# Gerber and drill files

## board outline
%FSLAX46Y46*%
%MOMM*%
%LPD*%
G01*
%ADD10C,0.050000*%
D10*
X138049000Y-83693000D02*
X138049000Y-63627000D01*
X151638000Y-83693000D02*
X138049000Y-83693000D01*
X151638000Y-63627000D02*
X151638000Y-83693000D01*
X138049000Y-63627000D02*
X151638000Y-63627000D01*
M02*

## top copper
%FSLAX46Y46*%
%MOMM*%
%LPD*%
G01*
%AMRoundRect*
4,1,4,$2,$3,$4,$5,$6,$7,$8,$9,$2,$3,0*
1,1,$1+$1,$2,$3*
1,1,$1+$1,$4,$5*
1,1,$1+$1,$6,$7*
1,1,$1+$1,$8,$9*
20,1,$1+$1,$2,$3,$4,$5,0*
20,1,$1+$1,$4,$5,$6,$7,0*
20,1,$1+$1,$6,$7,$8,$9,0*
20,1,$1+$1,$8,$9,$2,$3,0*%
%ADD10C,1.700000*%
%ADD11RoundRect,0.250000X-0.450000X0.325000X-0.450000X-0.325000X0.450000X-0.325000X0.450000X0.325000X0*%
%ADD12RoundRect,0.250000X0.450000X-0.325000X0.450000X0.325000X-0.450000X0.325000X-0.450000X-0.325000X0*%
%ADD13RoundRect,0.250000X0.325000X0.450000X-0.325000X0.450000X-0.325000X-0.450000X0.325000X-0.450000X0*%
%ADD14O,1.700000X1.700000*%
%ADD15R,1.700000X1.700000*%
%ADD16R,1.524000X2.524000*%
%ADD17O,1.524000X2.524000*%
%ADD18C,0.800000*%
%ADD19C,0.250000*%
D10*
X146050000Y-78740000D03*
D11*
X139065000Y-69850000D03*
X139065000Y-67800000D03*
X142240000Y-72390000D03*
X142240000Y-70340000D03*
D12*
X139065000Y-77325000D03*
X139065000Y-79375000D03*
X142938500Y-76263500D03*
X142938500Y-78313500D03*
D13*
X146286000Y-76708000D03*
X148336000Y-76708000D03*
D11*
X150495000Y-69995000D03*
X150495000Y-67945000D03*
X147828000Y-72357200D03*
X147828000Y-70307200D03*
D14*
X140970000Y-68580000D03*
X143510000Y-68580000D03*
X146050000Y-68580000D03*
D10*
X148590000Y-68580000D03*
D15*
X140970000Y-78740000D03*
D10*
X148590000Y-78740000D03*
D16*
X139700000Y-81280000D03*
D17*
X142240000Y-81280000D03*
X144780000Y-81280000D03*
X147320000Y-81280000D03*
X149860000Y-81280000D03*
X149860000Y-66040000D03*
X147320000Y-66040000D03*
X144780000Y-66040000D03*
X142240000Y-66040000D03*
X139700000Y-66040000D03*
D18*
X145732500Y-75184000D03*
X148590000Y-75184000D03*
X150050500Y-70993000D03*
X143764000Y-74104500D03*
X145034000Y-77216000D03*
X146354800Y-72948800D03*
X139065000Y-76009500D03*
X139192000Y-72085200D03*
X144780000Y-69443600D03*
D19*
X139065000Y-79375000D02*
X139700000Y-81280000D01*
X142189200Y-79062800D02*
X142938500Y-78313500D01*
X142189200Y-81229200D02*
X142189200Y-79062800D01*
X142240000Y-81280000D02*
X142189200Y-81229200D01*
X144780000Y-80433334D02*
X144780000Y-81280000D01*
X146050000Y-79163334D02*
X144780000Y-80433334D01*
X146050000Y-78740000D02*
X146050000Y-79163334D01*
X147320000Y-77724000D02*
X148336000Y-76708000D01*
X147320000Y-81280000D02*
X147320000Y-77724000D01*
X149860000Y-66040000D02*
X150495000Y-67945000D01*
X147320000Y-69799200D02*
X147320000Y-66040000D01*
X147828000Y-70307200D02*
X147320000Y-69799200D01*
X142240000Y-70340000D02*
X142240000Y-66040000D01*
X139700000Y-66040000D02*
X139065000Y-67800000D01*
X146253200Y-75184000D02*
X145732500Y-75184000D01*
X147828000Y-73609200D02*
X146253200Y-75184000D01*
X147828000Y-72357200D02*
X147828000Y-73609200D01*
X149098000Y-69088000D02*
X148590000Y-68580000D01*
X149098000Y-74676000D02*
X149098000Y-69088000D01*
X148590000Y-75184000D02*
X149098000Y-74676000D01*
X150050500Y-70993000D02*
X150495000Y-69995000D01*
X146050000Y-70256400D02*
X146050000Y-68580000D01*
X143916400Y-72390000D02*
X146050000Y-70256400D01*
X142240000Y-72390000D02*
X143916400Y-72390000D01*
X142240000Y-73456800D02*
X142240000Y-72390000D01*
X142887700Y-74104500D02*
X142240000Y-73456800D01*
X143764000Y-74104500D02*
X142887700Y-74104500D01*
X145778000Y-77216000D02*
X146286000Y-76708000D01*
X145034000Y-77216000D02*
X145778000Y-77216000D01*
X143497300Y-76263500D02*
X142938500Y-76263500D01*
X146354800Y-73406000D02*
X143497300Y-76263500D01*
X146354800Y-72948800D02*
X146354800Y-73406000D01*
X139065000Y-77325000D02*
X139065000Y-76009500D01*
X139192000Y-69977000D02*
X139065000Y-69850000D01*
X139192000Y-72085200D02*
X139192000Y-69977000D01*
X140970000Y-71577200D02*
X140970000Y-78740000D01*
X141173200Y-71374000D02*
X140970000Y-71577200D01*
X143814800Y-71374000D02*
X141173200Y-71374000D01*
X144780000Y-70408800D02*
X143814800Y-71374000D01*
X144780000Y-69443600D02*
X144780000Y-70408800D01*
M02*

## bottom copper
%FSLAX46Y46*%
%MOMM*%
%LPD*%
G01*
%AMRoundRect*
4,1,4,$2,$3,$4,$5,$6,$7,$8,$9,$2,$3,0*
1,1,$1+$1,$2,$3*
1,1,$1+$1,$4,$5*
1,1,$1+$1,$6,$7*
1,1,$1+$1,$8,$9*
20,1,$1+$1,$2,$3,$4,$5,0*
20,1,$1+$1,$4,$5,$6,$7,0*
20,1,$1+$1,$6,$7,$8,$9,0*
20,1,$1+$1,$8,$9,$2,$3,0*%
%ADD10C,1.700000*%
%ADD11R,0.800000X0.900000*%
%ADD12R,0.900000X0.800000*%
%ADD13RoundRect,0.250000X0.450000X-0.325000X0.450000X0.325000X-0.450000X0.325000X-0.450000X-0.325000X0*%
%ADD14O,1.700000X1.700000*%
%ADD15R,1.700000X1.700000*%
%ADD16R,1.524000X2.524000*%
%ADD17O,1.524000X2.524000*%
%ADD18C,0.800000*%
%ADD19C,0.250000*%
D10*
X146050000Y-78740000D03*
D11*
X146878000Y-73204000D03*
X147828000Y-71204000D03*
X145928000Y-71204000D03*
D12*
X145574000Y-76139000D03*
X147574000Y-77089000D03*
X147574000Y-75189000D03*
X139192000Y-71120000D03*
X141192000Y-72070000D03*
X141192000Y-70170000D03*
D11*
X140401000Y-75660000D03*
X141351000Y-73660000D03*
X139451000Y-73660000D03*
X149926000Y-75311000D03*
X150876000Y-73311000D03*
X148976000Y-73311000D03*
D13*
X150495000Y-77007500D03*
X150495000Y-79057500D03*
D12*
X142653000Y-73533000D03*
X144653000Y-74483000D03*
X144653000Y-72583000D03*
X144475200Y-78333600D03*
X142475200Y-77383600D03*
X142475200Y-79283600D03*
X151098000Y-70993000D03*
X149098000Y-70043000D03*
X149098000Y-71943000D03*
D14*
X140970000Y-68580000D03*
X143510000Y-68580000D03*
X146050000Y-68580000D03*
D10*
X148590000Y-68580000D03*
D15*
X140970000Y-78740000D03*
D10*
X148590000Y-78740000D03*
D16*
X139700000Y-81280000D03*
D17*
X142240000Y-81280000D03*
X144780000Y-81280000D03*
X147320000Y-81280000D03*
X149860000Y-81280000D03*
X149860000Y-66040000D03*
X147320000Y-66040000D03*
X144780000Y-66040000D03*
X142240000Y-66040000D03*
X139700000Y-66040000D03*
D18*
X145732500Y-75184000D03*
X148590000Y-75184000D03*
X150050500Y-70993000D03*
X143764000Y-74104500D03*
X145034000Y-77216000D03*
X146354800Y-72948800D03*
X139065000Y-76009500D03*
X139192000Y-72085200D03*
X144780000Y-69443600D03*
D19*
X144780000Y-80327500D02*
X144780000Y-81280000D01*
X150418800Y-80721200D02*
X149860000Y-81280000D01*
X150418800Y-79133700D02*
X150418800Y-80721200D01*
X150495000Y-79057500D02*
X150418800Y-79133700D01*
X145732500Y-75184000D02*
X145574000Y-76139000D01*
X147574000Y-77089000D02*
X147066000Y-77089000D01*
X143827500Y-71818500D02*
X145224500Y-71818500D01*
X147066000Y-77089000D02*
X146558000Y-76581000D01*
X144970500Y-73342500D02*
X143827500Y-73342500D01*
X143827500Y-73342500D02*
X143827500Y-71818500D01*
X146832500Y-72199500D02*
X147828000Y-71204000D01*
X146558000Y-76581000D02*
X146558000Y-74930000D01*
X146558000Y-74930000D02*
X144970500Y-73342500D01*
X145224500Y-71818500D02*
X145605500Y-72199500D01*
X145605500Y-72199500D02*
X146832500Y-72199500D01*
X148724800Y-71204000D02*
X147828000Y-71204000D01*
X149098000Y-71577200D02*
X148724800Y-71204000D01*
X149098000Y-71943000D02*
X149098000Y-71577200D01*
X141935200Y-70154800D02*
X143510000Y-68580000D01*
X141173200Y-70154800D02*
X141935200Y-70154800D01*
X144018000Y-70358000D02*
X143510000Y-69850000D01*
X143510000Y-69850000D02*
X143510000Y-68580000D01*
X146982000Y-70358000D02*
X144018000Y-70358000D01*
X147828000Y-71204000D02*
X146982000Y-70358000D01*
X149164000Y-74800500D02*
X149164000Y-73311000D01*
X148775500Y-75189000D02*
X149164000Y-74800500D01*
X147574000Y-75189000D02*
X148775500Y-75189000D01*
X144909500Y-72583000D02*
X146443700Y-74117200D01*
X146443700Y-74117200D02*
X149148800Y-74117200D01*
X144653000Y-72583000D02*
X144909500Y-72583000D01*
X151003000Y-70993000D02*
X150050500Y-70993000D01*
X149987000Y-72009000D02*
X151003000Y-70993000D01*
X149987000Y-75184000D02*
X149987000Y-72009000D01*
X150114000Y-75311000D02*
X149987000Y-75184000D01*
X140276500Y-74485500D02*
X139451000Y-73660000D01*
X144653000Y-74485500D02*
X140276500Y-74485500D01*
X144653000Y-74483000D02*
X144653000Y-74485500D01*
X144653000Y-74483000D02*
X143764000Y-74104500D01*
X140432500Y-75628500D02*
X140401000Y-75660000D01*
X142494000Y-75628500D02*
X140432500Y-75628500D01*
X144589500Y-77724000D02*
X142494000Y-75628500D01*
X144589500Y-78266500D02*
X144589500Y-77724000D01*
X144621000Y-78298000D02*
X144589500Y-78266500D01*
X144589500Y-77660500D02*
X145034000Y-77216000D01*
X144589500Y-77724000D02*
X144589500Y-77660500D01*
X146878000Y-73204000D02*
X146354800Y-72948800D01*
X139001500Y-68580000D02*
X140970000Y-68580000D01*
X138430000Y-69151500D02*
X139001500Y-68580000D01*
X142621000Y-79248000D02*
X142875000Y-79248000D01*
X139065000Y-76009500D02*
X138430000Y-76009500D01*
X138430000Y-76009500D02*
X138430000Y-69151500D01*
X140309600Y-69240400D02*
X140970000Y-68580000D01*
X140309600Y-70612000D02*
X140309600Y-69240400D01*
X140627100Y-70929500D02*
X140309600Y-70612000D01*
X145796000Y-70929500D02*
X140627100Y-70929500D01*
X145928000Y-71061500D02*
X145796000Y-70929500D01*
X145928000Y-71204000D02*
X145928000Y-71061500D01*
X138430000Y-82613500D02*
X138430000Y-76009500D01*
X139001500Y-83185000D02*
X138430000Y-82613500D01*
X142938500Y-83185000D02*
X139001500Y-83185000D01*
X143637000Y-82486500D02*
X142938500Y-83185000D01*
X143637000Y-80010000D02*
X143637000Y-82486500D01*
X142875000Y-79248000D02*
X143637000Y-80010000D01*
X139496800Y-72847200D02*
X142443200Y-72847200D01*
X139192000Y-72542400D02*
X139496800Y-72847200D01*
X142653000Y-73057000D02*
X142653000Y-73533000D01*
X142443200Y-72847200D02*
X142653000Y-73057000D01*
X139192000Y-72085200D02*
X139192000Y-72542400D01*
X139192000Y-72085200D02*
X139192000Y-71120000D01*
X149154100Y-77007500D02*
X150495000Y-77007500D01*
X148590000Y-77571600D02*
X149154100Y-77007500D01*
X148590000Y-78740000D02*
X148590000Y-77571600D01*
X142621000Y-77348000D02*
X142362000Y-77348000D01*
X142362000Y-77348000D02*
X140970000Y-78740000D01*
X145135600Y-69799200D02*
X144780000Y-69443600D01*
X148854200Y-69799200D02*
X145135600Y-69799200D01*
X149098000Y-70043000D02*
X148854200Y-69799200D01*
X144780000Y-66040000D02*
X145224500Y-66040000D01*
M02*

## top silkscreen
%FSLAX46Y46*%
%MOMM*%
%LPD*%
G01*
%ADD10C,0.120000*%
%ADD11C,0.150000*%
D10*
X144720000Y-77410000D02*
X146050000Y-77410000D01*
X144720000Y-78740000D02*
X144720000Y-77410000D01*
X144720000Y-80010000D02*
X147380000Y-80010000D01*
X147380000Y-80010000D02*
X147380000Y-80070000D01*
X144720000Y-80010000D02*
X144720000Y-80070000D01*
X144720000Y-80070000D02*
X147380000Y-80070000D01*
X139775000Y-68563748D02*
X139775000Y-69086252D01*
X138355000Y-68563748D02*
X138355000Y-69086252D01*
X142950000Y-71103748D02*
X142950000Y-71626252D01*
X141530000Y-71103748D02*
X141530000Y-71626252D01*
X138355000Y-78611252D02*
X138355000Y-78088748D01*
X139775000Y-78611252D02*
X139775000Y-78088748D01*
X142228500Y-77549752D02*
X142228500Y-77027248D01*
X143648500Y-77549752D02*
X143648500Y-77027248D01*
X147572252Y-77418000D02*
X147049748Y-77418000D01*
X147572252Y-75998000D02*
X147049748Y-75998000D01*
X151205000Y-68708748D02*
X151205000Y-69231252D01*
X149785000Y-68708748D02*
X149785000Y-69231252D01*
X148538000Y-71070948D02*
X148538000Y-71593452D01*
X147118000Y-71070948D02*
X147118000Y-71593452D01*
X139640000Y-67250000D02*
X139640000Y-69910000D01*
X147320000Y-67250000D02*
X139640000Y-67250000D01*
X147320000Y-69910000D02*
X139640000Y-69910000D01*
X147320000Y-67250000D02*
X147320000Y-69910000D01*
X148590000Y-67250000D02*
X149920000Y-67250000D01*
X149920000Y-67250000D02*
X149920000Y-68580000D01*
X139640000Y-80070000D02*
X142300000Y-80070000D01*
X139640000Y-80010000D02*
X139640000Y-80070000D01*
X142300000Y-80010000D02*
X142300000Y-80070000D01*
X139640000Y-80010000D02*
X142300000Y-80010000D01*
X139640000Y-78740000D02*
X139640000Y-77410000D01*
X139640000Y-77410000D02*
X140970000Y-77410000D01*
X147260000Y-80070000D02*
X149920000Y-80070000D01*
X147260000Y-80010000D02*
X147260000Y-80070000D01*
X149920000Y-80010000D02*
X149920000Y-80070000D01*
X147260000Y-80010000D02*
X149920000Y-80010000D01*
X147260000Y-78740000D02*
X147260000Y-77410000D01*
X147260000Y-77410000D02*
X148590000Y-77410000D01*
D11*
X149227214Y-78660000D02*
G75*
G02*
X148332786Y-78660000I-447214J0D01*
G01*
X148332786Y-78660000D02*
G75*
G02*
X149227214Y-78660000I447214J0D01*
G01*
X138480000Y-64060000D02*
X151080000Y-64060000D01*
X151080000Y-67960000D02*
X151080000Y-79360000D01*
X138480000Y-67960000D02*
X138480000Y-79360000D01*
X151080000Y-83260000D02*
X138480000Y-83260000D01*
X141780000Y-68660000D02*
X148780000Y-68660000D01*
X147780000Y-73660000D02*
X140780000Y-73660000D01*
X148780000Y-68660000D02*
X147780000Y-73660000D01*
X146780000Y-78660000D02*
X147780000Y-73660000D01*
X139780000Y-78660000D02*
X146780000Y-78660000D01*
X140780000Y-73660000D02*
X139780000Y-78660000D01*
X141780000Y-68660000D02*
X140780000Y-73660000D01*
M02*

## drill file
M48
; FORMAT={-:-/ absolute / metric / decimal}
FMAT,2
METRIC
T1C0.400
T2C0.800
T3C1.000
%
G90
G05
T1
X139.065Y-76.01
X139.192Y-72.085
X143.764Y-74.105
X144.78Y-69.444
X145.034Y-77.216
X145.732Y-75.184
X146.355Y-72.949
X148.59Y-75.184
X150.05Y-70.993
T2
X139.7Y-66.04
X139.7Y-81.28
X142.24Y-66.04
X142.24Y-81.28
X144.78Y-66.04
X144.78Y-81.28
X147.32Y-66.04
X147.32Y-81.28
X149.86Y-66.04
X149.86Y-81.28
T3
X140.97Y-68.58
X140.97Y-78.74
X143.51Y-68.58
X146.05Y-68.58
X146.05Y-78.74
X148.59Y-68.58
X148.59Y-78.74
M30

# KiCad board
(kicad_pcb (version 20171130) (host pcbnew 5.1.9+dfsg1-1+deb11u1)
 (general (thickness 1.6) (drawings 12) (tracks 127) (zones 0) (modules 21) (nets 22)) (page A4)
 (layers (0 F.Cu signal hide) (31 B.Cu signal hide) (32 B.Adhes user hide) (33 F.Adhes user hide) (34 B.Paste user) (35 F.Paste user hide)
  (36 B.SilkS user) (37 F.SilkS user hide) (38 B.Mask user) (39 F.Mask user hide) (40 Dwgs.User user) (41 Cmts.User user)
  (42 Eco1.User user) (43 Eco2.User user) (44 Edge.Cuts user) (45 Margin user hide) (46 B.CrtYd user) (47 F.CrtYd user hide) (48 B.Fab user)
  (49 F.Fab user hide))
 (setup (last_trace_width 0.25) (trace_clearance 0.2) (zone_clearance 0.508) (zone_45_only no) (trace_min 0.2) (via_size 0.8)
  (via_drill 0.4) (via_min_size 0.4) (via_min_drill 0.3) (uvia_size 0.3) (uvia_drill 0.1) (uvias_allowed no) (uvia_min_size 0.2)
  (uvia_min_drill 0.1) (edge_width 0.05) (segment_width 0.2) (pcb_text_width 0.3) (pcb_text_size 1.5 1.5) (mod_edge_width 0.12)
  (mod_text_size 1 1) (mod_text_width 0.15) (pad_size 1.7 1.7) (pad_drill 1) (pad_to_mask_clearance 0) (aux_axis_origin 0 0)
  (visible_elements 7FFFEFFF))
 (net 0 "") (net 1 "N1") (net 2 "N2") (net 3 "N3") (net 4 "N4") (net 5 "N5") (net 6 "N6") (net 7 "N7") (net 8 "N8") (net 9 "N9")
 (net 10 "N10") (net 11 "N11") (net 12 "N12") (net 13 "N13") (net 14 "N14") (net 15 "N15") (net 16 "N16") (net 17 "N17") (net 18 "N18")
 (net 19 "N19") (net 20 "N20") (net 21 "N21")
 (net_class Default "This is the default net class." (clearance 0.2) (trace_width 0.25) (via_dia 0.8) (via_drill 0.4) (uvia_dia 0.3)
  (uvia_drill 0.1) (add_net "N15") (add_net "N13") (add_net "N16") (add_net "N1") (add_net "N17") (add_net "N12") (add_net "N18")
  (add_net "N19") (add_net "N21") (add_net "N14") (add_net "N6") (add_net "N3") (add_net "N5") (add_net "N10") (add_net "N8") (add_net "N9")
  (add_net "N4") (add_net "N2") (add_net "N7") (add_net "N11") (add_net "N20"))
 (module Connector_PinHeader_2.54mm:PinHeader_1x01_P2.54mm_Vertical (layer F.Cu) (at 146.05 78.74)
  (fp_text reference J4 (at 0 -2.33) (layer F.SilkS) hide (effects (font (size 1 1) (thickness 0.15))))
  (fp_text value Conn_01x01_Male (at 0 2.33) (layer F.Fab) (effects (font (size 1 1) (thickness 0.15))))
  (fp_line (start -1.33 -1.33) (end 0 -1.33) (layer F.SilkS) (width 0.12))
  (fp_line (start -1.33 0) (end -1.33 -1.33) (layer F.SilkS) (width 0.12))
  (fp_line (start -1.33 1.27) (end 1.33 1.27) (layer F.SilkS) (width 0.12))
  (fp_line (start 1.33 1.27) (end 1.33 1.33) (layer F.SilkS) (width 0.12))
  (fp_line (start -1.33 1.27) (end -1.33 1.33) (layer F.SilkS) (width 0.12))
  (fp_line (start -1.33 1.33) (end 1.33 1.33) (layer F.SilkS) (width 0.12))
  (pad 1 thru_hole circle (at 0 0) (size 1.7 1.7) (drill 1) (layers *.Cu *.Mask) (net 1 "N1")))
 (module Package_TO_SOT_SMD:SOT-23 (layer B.Cu) (at 146.878 72.204 270)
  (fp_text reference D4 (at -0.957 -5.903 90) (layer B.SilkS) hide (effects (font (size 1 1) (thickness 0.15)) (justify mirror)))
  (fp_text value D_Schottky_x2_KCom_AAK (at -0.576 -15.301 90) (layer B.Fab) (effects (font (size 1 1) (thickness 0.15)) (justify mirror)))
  (pad 3 smd rect (at 1 0 270) (size 0.9 0.8) (layers B.Cu B.Paste B.Mask) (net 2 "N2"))
  (pad 2 smd rect (at -1 -0.95 270) (size 0.9 0.8) (layers B.Cu B.Paste B.Mask) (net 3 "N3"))
  (pad 1 smd rect (at -1 0.95 270) (size 0.9 0.8) (layers B.Cu B.Paste B.Mask) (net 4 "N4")))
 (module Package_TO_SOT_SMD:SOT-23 (layer B.Cu) (at 146.574 76.139 180)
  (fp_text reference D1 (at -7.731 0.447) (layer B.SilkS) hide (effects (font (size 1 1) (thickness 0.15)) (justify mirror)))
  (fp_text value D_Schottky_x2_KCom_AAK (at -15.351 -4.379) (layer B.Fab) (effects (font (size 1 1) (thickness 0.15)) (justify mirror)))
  (pad 3 smd rect (at 1 0 180) (size 0.9 0.8) (layers B.Cu B.Paste B.Mask) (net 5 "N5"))
  (pad 2 smd rect (at -1 -0.95 180) (size 0.9 0.8) (layers B.Cu B.Paste B.Mask) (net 3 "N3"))
  (pad 1 smd rect (at -1 0.95 180) (size 0.9 0.8) (layers B.Cu B.Paste B.Mask) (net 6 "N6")))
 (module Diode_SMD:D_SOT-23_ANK (layer B.Cu) (at 140.192 71.12 180)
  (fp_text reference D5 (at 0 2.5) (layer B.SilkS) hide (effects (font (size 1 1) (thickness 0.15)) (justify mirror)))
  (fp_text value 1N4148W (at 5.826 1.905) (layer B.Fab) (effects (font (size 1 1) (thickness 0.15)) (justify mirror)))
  (pad 1 smd rect (at 1 0 180) (size 0.9 0.8) (layers B.Cu B.Paste B.Mask) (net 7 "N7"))
  (pad "" smd rect (at -1 -0.95 180) (size 0.9 0.8) (layers B.Cu B.Paste B.Mask))
  (pad 2 smd rect (at -1 0.95 180) (size 0.9 0.8) (layers B.Cu B.Paste B.Mask) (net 3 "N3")))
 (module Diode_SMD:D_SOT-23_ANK (layer B.Cu) (at 140.401 74.66 270)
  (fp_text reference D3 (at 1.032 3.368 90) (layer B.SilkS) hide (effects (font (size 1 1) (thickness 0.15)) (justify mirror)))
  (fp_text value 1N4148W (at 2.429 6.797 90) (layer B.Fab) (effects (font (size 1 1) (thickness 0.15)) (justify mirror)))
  (pad 1 smd rect (at 1 0 270) (size 0.9 0.8) (layers B.Cu B.Paste B.Mask) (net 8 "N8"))
  (pad "" smd rect (at -1 -0.95 270) (size 0.9 0.8) (layers B.Cu B.Paste B.Mask))
  (pad 2 smd rect (at -1 0.95 270) (size 0.9 0.8) (layers B.Cu B.Paste B.Mask) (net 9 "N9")))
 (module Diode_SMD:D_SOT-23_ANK (layer B.Cu) (at 149.926 74.311 270)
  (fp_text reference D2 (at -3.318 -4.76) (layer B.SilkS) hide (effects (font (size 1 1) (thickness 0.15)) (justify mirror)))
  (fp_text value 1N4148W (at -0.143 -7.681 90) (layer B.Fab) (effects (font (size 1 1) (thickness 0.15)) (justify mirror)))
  (pad 1 smd rect (at 1 0 270) (size 0.9 0.8) (layers B.Cu B.Paste B.Mask) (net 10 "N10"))
  (pad "" smd rect (at -1 -0.95 270) (size 0.9 0.8) (layers B.Cu B.Paste B.Mask))
  (pad 2 smd rect (at -1 0.95 270) (size 0.9 0.8) (layers B.Cu B.Paste B.Mask) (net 6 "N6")))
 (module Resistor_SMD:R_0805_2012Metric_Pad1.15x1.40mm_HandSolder (layer B.Cu) (at 150.495 78.0325 90)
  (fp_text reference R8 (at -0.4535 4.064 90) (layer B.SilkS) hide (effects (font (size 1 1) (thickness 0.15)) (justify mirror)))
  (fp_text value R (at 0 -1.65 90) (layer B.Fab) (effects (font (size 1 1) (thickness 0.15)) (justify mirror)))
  (pad 2 smd roundrect (at 1.025 0 90) (size 1.15 1.4) (layers B.Cu B.Paste B.Mask) (roundrect_rratio 0.217391) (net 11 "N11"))
  (pad 1 smd roundrect (at -1.025 0 90) (size 1.15 1.4) (layers B.Cu B.Paste B.Mask) (roundrect_rratio 0.217391) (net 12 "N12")))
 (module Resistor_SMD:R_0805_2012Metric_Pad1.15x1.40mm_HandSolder (layer F.Cu) (at 139.065 68.825 270)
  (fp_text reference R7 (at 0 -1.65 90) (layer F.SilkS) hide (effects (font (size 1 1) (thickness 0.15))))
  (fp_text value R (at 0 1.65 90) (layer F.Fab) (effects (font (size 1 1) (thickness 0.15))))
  (fp_line (start -0.261252 -0.71) (end 0.261252 -0.71) (layer F.SilkS) (width 0.12))
  (fp_line (start -0.261252 0.71) (end 0.261252 0.71) (layer F.SilkS) (width 0.12))
  (pad 2 smd roundrect (at 1.025 0 270) (size 1.15 1.4) (layers F.Cu F.Paste F.Mask) (roundrect_rratio 0.217391) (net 7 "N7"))
  (pad 1 smd roundrect (at -1.025 0 270) (size 1.15 1.4) (layers F.Cu F.Paste F.Mask) (roundrect_rratio 0.217391) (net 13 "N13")))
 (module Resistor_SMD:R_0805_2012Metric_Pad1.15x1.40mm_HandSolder (layer F.Cu) (at 142.24 71.365 270)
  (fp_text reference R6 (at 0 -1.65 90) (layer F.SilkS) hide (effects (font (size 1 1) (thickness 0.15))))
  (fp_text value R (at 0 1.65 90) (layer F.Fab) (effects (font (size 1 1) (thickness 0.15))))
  (fp_line (start -0.261252 -0.71) (end 0.261252 -0.71) (layer F.SilkS) (width 0.12))
  (fp_line (start -0.261252 0.71) (end 0.261252 0.71) (layer F.SilkS) (width 0.12))
  (pad 2 smd roundrect (at 1.025 0 270) (size 1.15 1.4) (layers F.Cu F.Paste F.Mask) (roundrect_rratio 0.217391) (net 9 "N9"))
  (pad 1 smd roundrect (at -1.025 0 270) (size 1.15 1.4) (layers F.Cu F.Paste F.Mask) (roundrect_rratio 0.217391) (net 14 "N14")))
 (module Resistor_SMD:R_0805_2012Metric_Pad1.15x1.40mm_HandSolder (layer F.Cu) (at 139.065 78.35 90)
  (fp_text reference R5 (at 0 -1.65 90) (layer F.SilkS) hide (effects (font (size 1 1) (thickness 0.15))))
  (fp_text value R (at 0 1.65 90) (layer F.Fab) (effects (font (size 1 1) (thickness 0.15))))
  (fp_line (start -0.261252 -0.71) (end 0.261252 -0.71) (layer F.SilkS) (width 0.12))
  (fp_line (start -0.261252 0.71) (end 0.261252 0.71) (layer F.SilkS) (width 0.12))
  (pad 2 smd roundrect (at 1.025 0 90) (size 1.15 1.4) (layers F.Cu F.Paste F.Mask) (roundrect_rratio 0.217391) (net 4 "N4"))
  (pad 1 smd roundrect (at -1.025 0 90) (size 1.15 1.4) (layers F.Cu F.Paste F.Mask) (roundrect_rratio 0.217391) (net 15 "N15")))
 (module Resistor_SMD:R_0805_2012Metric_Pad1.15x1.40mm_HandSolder (layer F.Cu) (at 142.9385 77.2885 90)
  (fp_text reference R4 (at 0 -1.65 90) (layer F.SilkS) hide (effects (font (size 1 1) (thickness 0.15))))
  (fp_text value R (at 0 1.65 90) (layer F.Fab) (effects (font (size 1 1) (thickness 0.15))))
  (fp_line (start -0.261252 -0.71) (end 0.261252 -0.71) (layer F.SilkS) (width 0.12))
  (fp_line (start -0.261252 0.71) (end 0.261252 0.71) (layer F.SilkS) (width 0.12))
  (pad 2 smd roundrect (at 1.025 0 90) (size 1.15 1.4) (layers F.Cu F.Paste F.Mask) (roundrect_rratio 0.217391) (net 2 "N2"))
  (pad 1 smd roundrect (at -1.025 0 90) (size 1.15 1.4) (layers F.Cu F.Paste F.Mask) (roundrect_rratio 0.217391) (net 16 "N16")))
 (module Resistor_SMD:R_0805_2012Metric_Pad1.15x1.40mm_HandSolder (layer F.Cu) (at 147.311 76.708 180)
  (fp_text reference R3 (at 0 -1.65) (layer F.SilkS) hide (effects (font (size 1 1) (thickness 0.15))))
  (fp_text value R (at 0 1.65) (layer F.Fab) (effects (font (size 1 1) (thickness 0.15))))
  (fp_line (start -0.261252 -0.71) (end 0.261252 -0.71) (layer F.SilkS) (width 0.12))
  (fp_line (start -0.261252 0.71) (end 0.261252 0.71) (layer F.SilkS) (width 0.12))
  (pad 2 smd roundrect (at 1.025 0 180) (size 1.15 1.4) (layers F.Cu F.Paste F.Mask) (roundrect_rratio 0.217391) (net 8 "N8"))
  (pad 1 smd roundrect (at -1.025 0 180) (size 1.15 1.4) (layers F.Cu F.Paste F.Mask) (roundrect_rratio 0.217391) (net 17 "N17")))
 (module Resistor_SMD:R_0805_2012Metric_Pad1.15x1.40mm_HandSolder (layer F.Cu) (at 150.495 68.97 270)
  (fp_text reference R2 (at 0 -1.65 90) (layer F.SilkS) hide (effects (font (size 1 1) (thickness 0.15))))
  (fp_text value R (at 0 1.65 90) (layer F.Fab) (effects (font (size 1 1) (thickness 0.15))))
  (fp_line (start -0.261252 -0.71) (end 0.261252 -0.71) (layer F.SilkS) (width 0.12))
  (fp_line (start -0.261252 0.71) (end 0.261252 0.71) (layer F.SilkS) (width 0.12))
  (pad 2 smd roundrect (at 1.025 0 270) (size 1.15 1.4) (layers F.Cu F.Paste F.Mask) (roundrect_rratio 0.217391) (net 10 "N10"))
  (pad 1 smd roundrect (at -1.025 0 270) (size 1.15 1.4) (layers F.Cu F.Paste F.Mask) (roundrect_rratio 0.217391) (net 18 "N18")))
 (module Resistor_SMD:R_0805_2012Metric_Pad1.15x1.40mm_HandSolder (layer F.Cu) (at 147.828 71.3322 270)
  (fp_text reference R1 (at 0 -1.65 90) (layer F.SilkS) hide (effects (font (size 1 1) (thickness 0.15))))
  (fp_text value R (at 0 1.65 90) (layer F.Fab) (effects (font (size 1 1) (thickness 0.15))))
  (fp_line (start -0.261252 -0.71) (end 0.261252 -0.71) (layer F.SilkS) (width 0.12))
  (fp_line (start -0.261252 0.71) (end 0.261252 0.71) (layer F.SilkS) (width 0.12))
  (pad 2 smd roundrect (at 1.025 0 270) (size 1.15 1.4) (layers F.Cu F.Paste F.Mask) (roundrect_rratio 0.217391) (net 5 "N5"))
  (pad 1 smd roundrect (at -1.025 0 270) (size 1.15 1.4) (layers F.Cu F.Paste F.Mask) (roundrect_rratio 0.217391) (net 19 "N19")))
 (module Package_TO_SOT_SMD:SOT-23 (layer B.Cu) (at 143.653 73.533 180)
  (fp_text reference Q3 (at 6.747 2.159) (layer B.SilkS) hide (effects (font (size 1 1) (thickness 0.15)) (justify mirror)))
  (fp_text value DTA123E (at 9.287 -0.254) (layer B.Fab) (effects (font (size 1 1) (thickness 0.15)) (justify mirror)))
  (pad 3 smd rect (at 1 0 180) (size 0.9 0.8) (layers B.Cu B.Paste B.Mask) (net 7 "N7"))
  (pad 2 smd rect (at -1 -0.95 180) (size 0.9 0.8) (layers B.Cu B.Paste B.Mask) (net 9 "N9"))
  (pad 1 smd rect (at -1 0.95 180) (size 0.9 0.8) (layers B.Cu B.Paste B.Mask) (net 6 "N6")))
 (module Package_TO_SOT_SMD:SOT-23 (layer B.Cu) (at 143.4752 78.3336)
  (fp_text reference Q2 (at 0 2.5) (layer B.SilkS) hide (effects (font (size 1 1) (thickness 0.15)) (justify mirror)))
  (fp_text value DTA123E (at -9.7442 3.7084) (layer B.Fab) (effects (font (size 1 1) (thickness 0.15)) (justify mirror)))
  (pad 3 smd rect (at 1 0) (size 0.9 0.8) (layers B.Cu B.Paste B.Mask) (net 8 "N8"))
  (pad 2 smd rect (at -1 -0.95) (size 0.9 0.8) (layers B.Cu B.Paste B.Mask) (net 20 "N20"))
  (pad 1 smd rect (at -1 0.95) (size 0.9 0.8) (layers B.Cu B.Paste B.Mask) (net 4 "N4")))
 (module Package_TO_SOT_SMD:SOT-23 (layer B.Cu) (at 150.098 70.993)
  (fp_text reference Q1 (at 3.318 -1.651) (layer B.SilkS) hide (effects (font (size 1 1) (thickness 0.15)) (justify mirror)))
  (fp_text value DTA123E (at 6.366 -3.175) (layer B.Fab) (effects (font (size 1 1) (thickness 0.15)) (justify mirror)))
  (pad 3 smd rect (at 1 0) (size 0.9 0.8) (layers B.Cu B.Paste B.Mask) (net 10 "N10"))
  (pad 2 smd rect (at -1 -0.95) (size 0.9 0.8) (layers B.Cu B.Paste B.Mask) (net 20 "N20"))
  (pad 1 smd rect (at -1 0.95) (size 0.9 0.8) (layers B.Cu B.Paste B.Mask) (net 3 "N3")))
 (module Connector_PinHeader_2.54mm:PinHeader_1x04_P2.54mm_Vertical (layer F.Cu) (at 148.59 68.58 270)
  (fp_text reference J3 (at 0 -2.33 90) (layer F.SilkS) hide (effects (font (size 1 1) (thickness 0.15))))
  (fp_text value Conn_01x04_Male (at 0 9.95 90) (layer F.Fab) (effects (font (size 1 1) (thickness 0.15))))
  (fp_line (start -1.33 8.95) (end 1.33 8.95) (layer F.SilkS) (width 0.12))
  (fp_line (start -1.33 1.27) (end -1.33 8.95) (layer F.SilkS) (width 0.12))
  (fp_line (start 1.33 1.27) (end 1.33 8.95) (layer F.SilkS) (width 0.12))
  (fp_line (start -1.33 1.27) (end 1.33 1.27) (layer F.SilkS) (width 0.12))
  (fp_line (start -1.33 0) (end -1.33 -1.33) (layer F.SilkS) (width 0.12))
  (fp_line (start -1.33 -1.33) (end 0 -1.33) (layer F.SilkS) (width 0.12))
  (pad 4 thru_hole oval (at 0 7.62 270) (size 1.7 1.7) (drill 1) (layers *.Cu *.Mask) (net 4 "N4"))
  (pad 3 thru_hole oval (at 0 5.08 270) (size 1.7 1.7) (drill 1) (layers *.Cu *.Mask) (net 3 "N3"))
  (pad 2 thru_hole oval (at 0 2.54 270) (size 1.7 1.7) (drill 1) (layers *.Cu *.Mask) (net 9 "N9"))
  (pad 1 thru_hole circle (at 0 0 270) (size 1.7 1.7) (drill 1) (layers *.Cu *.Mask) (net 6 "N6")))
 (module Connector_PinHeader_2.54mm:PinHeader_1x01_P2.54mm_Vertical (layer F.Cu) (at 140.97 78.74)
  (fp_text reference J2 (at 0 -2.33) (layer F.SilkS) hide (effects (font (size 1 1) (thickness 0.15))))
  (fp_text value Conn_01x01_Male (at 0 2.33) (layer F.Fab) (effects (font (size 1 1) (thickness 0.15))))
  (fp_line (start -1.33 1.33) (end 1.33 1.33) (layer F.SilkS) (width 0.12))
  (fp_line (start -1.33 1.27) (end -1.33 1.33) (layer F.SilkS) (width 0.12))
  (fp_line (start 1.33 1.27) (end 1.33 1.33) (layer F.SilkS) (width 0.12))
  (fp_line (start -1.33 1.27) (end 1.33 1.27) (layer F.SilkS) (width 0.12))
  (fp_line (start -1.33 0) (end -1.33 -1.33) (layer F.SilkS) (width 0.12))
  (fp_line (start -1.33 -1.33) (end 0 -1.33) (layer F.SilkS) (width 0.12))
  (pad 1 thru_hole rect (at 0 0) (size 1.7 1.7) (drill 1) (layers *.Cu *.Mask) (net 20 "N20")))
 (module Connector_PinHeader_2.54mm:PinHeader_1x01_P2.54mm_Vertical (layer F.Cu) (at 148.59 78.74)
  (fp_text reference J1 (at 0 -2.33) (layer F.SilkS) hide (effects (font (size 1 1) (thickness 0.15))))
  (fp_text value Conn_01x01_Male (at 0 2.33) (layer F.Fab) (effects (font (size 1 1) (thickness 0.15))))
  (fp_line (start -1.33 1.33) (end 1.33 1.33) (layer F.SilkS) (width 0.12))
  (fp_line (start -1.33 1.27) (end -1.33 1.33) (layer F.SilkS) (width 0.12))
  (fp_line (start 1.33 1.27) (end 1.33 1.33) (layer F.SilkS) (width 0.12))
  (fp_line (start -1.33 1.27) (end 1.33 1.27) (layer F.SilkS) (width 0.12))
  (fp_line (start -1.33 0) (end -1.33 -1.33) (layer F.SilkS) (width 0.12))
  (fp_line (start -1.33 -1.33) (end 0 -1.33) (layer F.SilkS) (width 0.12))
  (pad 1 thru_hole circle (at 0 0) (size 1.7 1.7) (drill 1) (layers *.Cu *.Mask) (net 11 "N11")))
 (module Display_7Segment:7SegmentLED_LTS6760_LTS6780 (layer F.Cu) (at 139.7 81.28 90)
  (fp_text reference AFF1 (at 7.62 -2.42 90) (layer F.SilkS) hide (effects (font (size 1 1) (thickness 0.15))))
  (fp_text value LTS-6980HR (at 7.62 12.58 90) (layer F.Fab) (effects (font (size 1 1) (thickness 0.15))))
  (fp_circle (center 2.62 9.08) (end 2.42 9.48) (layer F.SilkS) (width 0.15))
  (fp_line (start 17.22 -1.22) (end 17.22 11.38) (layer F.SilkS) (width 0.15))
  (fp_line (start 13.32 11.38) (end 1.92 11.38) (layer F.SilkS) (width 0.15))
  (fp_line (start 13.32 -1.22) (end 1.92 -1.22) (layer F.SilkS) (width 0.15))
  (fp_line (start -1.98 11.38) (end -1.98 -1.22) (layer F.SilkS) (width 0.15))
  (fp_line (start 12.62 2.08) (end 12.62 9.08) (layer F.SilkS) (width 0.15))
  (fp_line (start 7.62 8.08) (end 7.62 1.08) (layer F.SilkS) (width 0.15))
  (fp_line (start 12.62 9.08) (end 7.62 8.08) (layer F.SilkS) (width 0.15))
  (fp_line (start 2.62 7.08) (end 7.62 8.08) (layer F.SilkS) (width 0.15))
  (fp_line (start 2.62 0.08) (end 2.62 7.08) (layer F.SilkS) (width 0.15))
  (fp_line (start 7.62 1.08) (end 2.62 0.08) (layer F.SilkS) (width 0.15))
  (fp_line (start 12.62 2.08) (end 7.62 1.08) (layer F.SilkS) (width 0.15))
  (pad 1 thru_hole rect (at 0 0) (size 1.524 2.524) (drill 0.8) (layers *.Cu *.Mask) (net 15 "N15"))
  (pad 2 thru_hole oval (at 0 2.54) (size 1.524 2.524) (drill 0.8) (layers *.Cu *.Mask) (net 16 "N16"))
  (pad 3 thru_hole oval (at 0 5.08) (size 1.524 2.524) (drill 0.8) (layers *.Cu *.Mask) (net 1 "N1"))
  (pad 4 thru_hole oval (at 0 7.62) (size 1.524 2.524) (drill 0.8) (layers *.Cu *.Mask) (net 17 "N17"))
  (pad 5 thru_hole oval (at 0 10.16) (size 1.524 2.524) (drill 0.8) (layers *.Cu *.Mask) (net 12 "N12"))
  (pad 6 thru_hole oval (at 15.24 10.16) (size 1.524 2.524) (drill 0.8) (layers *.Cu *.Mask) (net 18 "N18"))
  (pad 7 thru_hole oval (at 15.24 7.62) (size 1.524 2.524) (drill 0.8) (layers *.Cu *.Mask) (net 19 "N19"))
  (pad 8 thru_hole oval (at 15.24 5.08) (size 1.524 2.524) (drill 0.8) (layers *.Cu *.Mask) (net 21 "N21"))
  (pad 9 thru_hole oval (at 15.24 2.54) (size 1.524 2.524) (drill 0.8) (layers *.Cu *.Mask) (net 14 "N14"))
  (pad 10 thru_hole oval (at 15.24 0) (size 1.524 2.524) (drill 0.8) (layers *.Cu *.Mask) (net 13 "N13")))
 (gr_line (start 138.049 83.693) (end 138.049 63.627) (layer Edge.Cuts) (width 0.05))
 (gr_line (start 151.638 83.693) (end 138.049 83.693) (layer Edge.Cuts) (width 0.05))
 (gr_line (start 151.638 63.627) (end 151.638 83.693) (layer Edge.Cuts) (width 0.05))
 (gr_line (start 138.049 63.627) (end 151.638 63.627) (layer Edge.Cuts) (width 0.05))
 (segment (start 139.065 79.375) (end 139.7 81.28) (width 0.25) (layer F.Cu) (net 15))
 (segment (start 142.1892 79.0628) (end 142.9385 78.3135) (width 0.25) (layer F.Cu) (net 16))
 (segment (start 142.1892 81.2292) (end 142.1892 79.0628) (width 0.25) (layer F.Cu) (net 16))
 (segment (start 142.24 81.28) (end 142.1892 81.2292) (width 0.25) (layer F.Cu) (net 16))
 (segment (start 144.78 80.3275) (end 144.78 81.28) (width 0.25) (layer B.Cu) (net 1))
 (segment (start 144.78 80.433334) (end 144.78 81.28) (width 0.25) (layer F.Cu) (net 1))
 (segment (start 146.05 79.163334) (end 144.78 80.433334) (width 0.25) (layer F.Cu) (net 1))
 (segment (start 146.05 78.74) (end 146.05 79.163334) (width 0.25) (layer F.Cu) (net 1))
 (segment (start 147.32 77.724) (end 148.336 76.708) (width 0.25) (layer F.Cu) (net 17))
 (segment (start 147.32 81.28) (end 147.32 77.724) (width 0.25) (layer F.Cu) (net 17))
 (segment (start 150.4188 80.7212) (end 149.86 81.28) (width 0.25) (layer B.Cu) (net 12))
 (segment (start 150.4188 79.1337) (end 150.4188 80.7212) (width 0.25) (layer B.Cu) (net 12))
 (segment (start 150.495 79.0575) (end 150.4188 79.1337) (width 0.25) (layer B.Cu) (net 12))
 (segment (start 149.86 66.04) (end 150.495 67.945) (width 0.25) (layer F.Cu) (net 18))
 (segment (start 147.32 69.7992) (end 147.32 66.04) (width 0.25) (layer F.Cu) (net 19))
 (segment (start 147.828 70.3072) (end 147.32 69.7992) (width 0.25) (layer F.Cu) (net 19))
 (segment (start 142.24 70.34) (end 142.24 66.04) (width 0.25) (layer F.Cu) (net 14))
 (segment (start 139.7 66.04) (end 139.065 67.8) (width 0.25) (layer F.Cu) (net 13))
 (via (at 145.7325 75.184) (size 0.8) (drill 0.4) (layers F.Cu B.Cu) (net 5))
 (segment (start 145.7325 75.184) (end 145.574 76.139) (width 0.25) (layer B.Cu) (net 5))
 (segment (start 146.2532 75.184) (end 145.7325 75.184) (width 0.25) (layer F.Cu) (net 5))
 (segment (start 147.828 73.6092) (end 146.2532 75.184) (width 0.25) (layer F.Cu) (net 5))
 (segment (start 147.828 72.3572) (end 147.828 73.6092) (width 0.25) (layer F.Cu) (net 5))
 (segment (start 147.574 77.089) (end 147.066 77.089) (width 0.25) (layer B.Cu) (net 3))
 (segment (start 143.8275 71.8185) (end 145.2245 71.8185) (width 0.25) (layer B.Cu) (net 3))
 (segment (start 147.066 77.089) (end 146.558 76.581) (width 0.25) (layer B.Cu) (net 3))
 (segment (start 144.9705 73.3425) (end 143.8275 73.3425) (width 0.25) (layer B.Cu) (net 3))
 (segment (start 143.8275 73.3425) (end 143.8275 71.8185) (width 0.25) (layer B.Cu) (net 3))
 (segment (start 146.8325 72.1995) (end 147.828 71.204) (width 0.25) (layer B.Cu) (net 3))
 (segment (start 146.558 76.581) (end 146.558 74.93) (width 0.25) (layer B.Cu) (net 3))
 (segment (start 146.558 74.93) (end 144.9705 73.3425) (width 0.25) (layer B.Cu) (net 3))
 (segment (start 145.2245 71.8185) (end 145.6055 72.1995) (width 0.25) (layer B.Cu) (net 3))
 (segment (start 145.6055 72.1995) (end 146.8325 72.1995) (width 0.25) (layer B.Cu) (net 3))
 (segment (start 148.7248 71.204) (end 147.828 71.204) (width 0.25) (layer B.Cu) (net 3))
 (segment (start 149.098 71.5772) (end 148.7248 71.204) (width 0.25) (layer B.Cu) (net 3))
 (segment (start 149.098 71.943) (end 149.098 71.5772) (width 0.25) (layer B.Cu) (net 3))
 (segment (start 141.9352 70.1548) (end 143.51 68.58) (width 0.25) (layer B.Cu) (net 3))
 (segment (start 141.1732 70.1548) (end 141.9352 70.1548) (width 0.25) (layer B.Cu) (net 3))
 (segment (start 144.018 70.358) (end 143.51 69.85) (width 0.25) (layer B.Cu) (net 3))
 (segment (start 143.51 69.85) (end 143.51 68.58) (width 0.25) (layer B.Cu) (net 3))
 (segment (start 146.982 70.358) (end 144.018 70.358) (width 0.25) (layer B.Cu) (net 3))
 (segment (start 147.828 71.204) (end 146.982 70.358) (width 0.25) (layer B.Cu) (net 3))
 (segment (start 149.164 74.8005) (end 149.164 73.311) (width 0.25) (layer B.Cu) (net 6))
 (segment (start 148.7755 75.189) (end 149.164 74.8005) (width 0.25) (layer B.Cu) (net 6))
 (segment (start 147.574 75.189) (end 148.7755 75.189) (width 0.25) (layer B.Cu) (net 6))
 (segment (start 144.9095 72.583) (end 146.4437 74.1172) (width 0.25) (layer B.Cu) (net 6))
 (segment (start 146.4437 74.1172) (end 149.1488 74.1172) (width 0.25) (layer B.Cu) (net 6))
 (segment (start 144.653 72.583) (end 144.9095 72.583) (width 0.25) (layer B.Cu) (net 6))
 (segment (start 149.098 69.088) (end 148.59 68.58) (width 0.25) (layer F.Cu) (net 6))
 (segment (start 149.098 74.676) (end 149.098 69.088) (width 0.25) (layer F.Cu) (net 6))
 (segment (start 148.59 75.184) (end 149.098 74.676) (width 0.25) (layer F.Cu) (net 6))
 (via (at 148.59 75.184) (size 0.8) (drill 0.4) (layers F.Cu B.Cu) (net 6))
 (via (at 150.0505 70.993) (size 0.8) (drill 0.4) (layers F.Cu B.Cu) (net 10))
 (segment (start 151.003 70.993) (end 150.0505 70.993) (width 0.25) (layer B.Cu) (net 10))
 (segment (start 150.0505 70.993) (end 150.495 69.995) (width 0.25) (layer F.Cu) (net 10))
 (segment (start 149.987 72.009) (end 151.003 70.993) (width 0.25) (layer B.Cu) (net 10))
 (segment (start 149.987 75.184) (end 149.987 72.009) (width 0.25) (layer B.Cu) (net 10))
 (segment (start 150.114 75.311) (end 149.987 75.184) (width 0.25) (layer B.Cu) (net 10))
 (segment (start 140.2765 74.4855) (end 139.451 73.66) (width 0.25) (layer B.Cu) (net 9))
 (segment (start 144.653 74.4855) (end 140.2765 74.4855) (width 0.25) (layer B.Cu) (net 9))
 (segment (start 144.653 74.483) (end 144.653 74.4855) (width 0.25) (layer B.Cu) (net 9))
 (via (at 143.764 74.1045) (size 0.8) (drill 0.4) (layers F.Cu B.Cu) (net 9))
 (segment (start 144.653 74.483) (end 143.764 74.1045) (width 0.25) (layer B.Cu) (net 9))
 (segment (start 146.05 70.2564) (end 146.05 68.58) (width 0.25) (layer F.Cu) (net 9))
 (segment (start 143.9164 72.39) (end 146.05 70.2564) (width 0.25) (layer F.Cu) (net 9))
 (segment (start 142.24 72.39) (end 143.9164 72.39) (width 0.25) (layer F.Cu) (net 9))
 (segment (start 142.24 73.4568) (end 142.24 72.39) (width 0.25) (layer F.Cu) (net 9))
 (segment (start 142.8877 74.1045) (end 142.24 73.4568) (width 0.25) (layer F.Cu) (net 9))
 (segment (start 143.764 74.1045) (end 142.8877 74.1045) (width 0.25) (layer F.Cu) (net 9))
 (segment (start 140.4325 75.6285) (end 140.401 75.66) (width 0.25) (layer B.Cu) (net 8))
 (segment (start 142.494 75.6285) (end 140.4325 75.6285) (width 0.25) (layer B.Cu) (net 8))
 (segment (start 144.5895 77.724) (end 142.494 75.6285) (width 0.25) (layer B.Cu) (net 8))
 (segment (start 144.5895 78.2665) (end 144.5895 77.724) (width 0.25) (layer B.Cu) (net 8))
 (segment (start 144.621 78.298) (end 144.5895 78.2665) (width 0.25) (layer B.Cu) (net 8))
 (segment (start 144.5895 77.6605) (end 145.034 77.216) (width 0.25) (layer B.Cu) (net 8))
 (segment (start 145.778 77.216) (end 146.286 76.708) (width 0.25) (layer F.Cu) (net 8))
 (segment (start 145.034 77.216) (end 145.778 77.216) (width 0.25) (layer F.Cu) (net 8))
 (segment (start 144.5895 77.724) (end 144.5895 77.6605) (width 0.25) (layer B.Cu) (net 8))
 (via (at 145.034 77.216) (size 0.8) (drill 0.4) (layers F.Cu B.Cu) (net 8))
 (via (at 146.3548 72.9488) (size 0.8) (drill 0.4) (layers F.Cu B.Cu) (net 2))
 (segment (start 143.4973 76.2635) (end 142.9385 76.2635) (width 0.25) (layer F.Cu) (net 2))
 (segment (start 146.3548 73.406) (end 143.4973 76.2635) (width 0.25) (layer F.Cu) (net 2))
 (segment (start 146.3548 72.9488) (end 146.3548 73.406) (width 0.25) (layer F.Cu) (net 2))
 (segment (start 146.878 73.204) (end 146.3548 72.9488) (width 0.25) (layer B.Cu) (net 2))
 (segment (start 139.0015 68.58) (end 140.97 68.58) (width 0.25) (layer B.Cu) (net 4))
 (segment (start 138.43 69.1515) (end 139.0015 68.58) (width 0.25) (layer B.Cu) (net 4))
 (segment (start 142.621 79.248) (end 142.875 79.248) (width 0.25) (layer B.Cu) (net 4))
 (via (at 139.065 76.0095) (size 0.8) (drill 0.4) (layers F.Cu B.Cu) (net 4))
 (segment (start 139.065 77.325) (end 139.065 76.0095) (width 0.25) (layer F.Cu) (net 4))
 (segment (start 139.065 76.0095) (end 138.43 76.0095) (width 0.25) (layer B.Cu) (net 4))
 (segment (start 138.43 76.0095) (end 138.43 69.1515) (width 0.25) (layer B.Cu) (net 4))
 (segment (start 140.3096 69.2404) (end 140.97 68.58) (width 0.25) (layer B.Cu) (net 4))
 (segment (start 140.3096 70.612) (end 140.3096 69.2404) (width 0.25) (layer B.Cu) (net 4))
 (segment (start 140.6271 70.9295) (end 140.3096 70.612) (width 0.25) (layer B.Cu) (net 4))
 (segment (start 145.796 70.9295) (end 140.6271 70.9295) (width 0.25) (layer B.Cu) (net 4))
 (segment (start 145.928 71.0615) (end 145.796 70.9295) (width 0.25) (layer B.Cu) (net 4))
 (segment (start 145.928 71.204) (end 145.928 71.0615) (width 0.25) (layer B.Cu) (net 4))
 (segment (start 138.43 82.6135) (end 138.43 76.0095) (width 0.25) (layer B.Cu) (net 4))
 (segment (start 139.0015 83.185) (end 138.43 82.6135) (width 0.25) (layer B.Cu) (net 4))
 (segment (start 142.9385 83.185) (end 139.0015 83.185) (width 0.25) (layer B.Cu) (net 4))
 (segment (start 143.637 82.4865) (end 142.9385 83.185) (width 0.25) (layer B.Cu) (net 4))
 (segment (start 143.637 80.01) (end 143.637 82.4865) (width 0.25) (layer B.Cu) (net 4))
 (segment (start 142.875 79.248) (end 143.637 80.01) (width 0.25) (layer B.Cu) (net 4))
 (segment (start 139.4968 72.8472) (end 142.4432 72.8472) (width 0.25) (layer B.Cu) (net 7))
 (segment (start 139.192 72.5424) (end 139.4968 72.8472) (width 0.25) (layer B.Cu) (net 7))
 (segment (start 139.192 69.977) (end 139.065 69.85) (width 0.25) (layer F.Cu) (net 7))
 (segment (start 142.653 73.057) (end 142.653 73.533) (width 0.25) (layer B.Cu) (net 7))
 (segment (start 142.4432 72.8472) (end 142.653 73.057) (width 0.25) (layer B.Cu) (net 7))
 (segment (start 139.192 72.0852) (end 139.192 72.5424) (width 0.25) (layer B.Cu) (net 7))
 (segment (start 139.192 72.0852) (end 139.192 69.977) (width 0.25) (layer F.Cu) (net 7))
 (via (at 139.192 72.0852) (size 0.8) (drill 0.4) (layers F.Cu B.Cu) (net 7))
 (segment (start 139.192 72.0852) (end 139.192 71.12) (width 0.25) (layer B.Cu) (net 7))
 (segment (start 149.1541 77.0075) (end 150.495 77.0075) (width 0.25) (layer B.Cu) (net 11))
 (segment (start 148.59 77.5716) (end 149.1541 77.0075) (width 0.25) (layer B.Cu) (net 11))
 (segment (start 148.59 78.74) (end 148.59 77.5716) (width 0.25) (layer B.Cu) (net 11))
 (segment (start 142.621 77.348) (end 142.362 77.348) (width 0.25) (layer B.Cu) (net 20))
 (segment (start 142.362 77.348) (end 140.97 78.74) (width 0.25) (layer B.Cu) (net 20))
 (via (at 144.78 69.4436) (size 0.8) (drill 0.4) (layers F.Cu B.Cu) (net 20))
 (segment (start 140.97 71.5772) (end 140.97 78.74) (width 0.25) (layer F.Cu) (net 20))
 (segment (start 141.1732 71.374) (end 140.97 71.5772) (width 0.25) (layer F.Cu) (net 20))
 (segment (start 143.8148 71.374) (end 141.1732 71.374) (width 0.25) (layer F.Cu) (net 20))
 (segment (start 144.78 70.4088) (end 143.8148 71.374) (width 0.25) (layer F.Cu) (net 20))
 (segment (start 144.78 69.4436) (end 144.78 70.4088) (width 0.25) (layer F.Cu) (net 20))
 (segment (start 145.1356 69.7992) (end 144.78 69.4436) (width 0.25) (layer B.Cu) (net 20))
 (segment (start 148.8542 69.7992) (end 145.1356 69.7992) (width 0.25) (layer B.Cu) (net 20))
 (segment (start 149.098 70.043) (end 148.8542 69.7992) (width 0.25) (layer B.Cu) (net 20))
 (segment (start 144.78 66.04) (end 145.2245 66.04) (width 0.25) (layer B.Cu) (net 21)))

